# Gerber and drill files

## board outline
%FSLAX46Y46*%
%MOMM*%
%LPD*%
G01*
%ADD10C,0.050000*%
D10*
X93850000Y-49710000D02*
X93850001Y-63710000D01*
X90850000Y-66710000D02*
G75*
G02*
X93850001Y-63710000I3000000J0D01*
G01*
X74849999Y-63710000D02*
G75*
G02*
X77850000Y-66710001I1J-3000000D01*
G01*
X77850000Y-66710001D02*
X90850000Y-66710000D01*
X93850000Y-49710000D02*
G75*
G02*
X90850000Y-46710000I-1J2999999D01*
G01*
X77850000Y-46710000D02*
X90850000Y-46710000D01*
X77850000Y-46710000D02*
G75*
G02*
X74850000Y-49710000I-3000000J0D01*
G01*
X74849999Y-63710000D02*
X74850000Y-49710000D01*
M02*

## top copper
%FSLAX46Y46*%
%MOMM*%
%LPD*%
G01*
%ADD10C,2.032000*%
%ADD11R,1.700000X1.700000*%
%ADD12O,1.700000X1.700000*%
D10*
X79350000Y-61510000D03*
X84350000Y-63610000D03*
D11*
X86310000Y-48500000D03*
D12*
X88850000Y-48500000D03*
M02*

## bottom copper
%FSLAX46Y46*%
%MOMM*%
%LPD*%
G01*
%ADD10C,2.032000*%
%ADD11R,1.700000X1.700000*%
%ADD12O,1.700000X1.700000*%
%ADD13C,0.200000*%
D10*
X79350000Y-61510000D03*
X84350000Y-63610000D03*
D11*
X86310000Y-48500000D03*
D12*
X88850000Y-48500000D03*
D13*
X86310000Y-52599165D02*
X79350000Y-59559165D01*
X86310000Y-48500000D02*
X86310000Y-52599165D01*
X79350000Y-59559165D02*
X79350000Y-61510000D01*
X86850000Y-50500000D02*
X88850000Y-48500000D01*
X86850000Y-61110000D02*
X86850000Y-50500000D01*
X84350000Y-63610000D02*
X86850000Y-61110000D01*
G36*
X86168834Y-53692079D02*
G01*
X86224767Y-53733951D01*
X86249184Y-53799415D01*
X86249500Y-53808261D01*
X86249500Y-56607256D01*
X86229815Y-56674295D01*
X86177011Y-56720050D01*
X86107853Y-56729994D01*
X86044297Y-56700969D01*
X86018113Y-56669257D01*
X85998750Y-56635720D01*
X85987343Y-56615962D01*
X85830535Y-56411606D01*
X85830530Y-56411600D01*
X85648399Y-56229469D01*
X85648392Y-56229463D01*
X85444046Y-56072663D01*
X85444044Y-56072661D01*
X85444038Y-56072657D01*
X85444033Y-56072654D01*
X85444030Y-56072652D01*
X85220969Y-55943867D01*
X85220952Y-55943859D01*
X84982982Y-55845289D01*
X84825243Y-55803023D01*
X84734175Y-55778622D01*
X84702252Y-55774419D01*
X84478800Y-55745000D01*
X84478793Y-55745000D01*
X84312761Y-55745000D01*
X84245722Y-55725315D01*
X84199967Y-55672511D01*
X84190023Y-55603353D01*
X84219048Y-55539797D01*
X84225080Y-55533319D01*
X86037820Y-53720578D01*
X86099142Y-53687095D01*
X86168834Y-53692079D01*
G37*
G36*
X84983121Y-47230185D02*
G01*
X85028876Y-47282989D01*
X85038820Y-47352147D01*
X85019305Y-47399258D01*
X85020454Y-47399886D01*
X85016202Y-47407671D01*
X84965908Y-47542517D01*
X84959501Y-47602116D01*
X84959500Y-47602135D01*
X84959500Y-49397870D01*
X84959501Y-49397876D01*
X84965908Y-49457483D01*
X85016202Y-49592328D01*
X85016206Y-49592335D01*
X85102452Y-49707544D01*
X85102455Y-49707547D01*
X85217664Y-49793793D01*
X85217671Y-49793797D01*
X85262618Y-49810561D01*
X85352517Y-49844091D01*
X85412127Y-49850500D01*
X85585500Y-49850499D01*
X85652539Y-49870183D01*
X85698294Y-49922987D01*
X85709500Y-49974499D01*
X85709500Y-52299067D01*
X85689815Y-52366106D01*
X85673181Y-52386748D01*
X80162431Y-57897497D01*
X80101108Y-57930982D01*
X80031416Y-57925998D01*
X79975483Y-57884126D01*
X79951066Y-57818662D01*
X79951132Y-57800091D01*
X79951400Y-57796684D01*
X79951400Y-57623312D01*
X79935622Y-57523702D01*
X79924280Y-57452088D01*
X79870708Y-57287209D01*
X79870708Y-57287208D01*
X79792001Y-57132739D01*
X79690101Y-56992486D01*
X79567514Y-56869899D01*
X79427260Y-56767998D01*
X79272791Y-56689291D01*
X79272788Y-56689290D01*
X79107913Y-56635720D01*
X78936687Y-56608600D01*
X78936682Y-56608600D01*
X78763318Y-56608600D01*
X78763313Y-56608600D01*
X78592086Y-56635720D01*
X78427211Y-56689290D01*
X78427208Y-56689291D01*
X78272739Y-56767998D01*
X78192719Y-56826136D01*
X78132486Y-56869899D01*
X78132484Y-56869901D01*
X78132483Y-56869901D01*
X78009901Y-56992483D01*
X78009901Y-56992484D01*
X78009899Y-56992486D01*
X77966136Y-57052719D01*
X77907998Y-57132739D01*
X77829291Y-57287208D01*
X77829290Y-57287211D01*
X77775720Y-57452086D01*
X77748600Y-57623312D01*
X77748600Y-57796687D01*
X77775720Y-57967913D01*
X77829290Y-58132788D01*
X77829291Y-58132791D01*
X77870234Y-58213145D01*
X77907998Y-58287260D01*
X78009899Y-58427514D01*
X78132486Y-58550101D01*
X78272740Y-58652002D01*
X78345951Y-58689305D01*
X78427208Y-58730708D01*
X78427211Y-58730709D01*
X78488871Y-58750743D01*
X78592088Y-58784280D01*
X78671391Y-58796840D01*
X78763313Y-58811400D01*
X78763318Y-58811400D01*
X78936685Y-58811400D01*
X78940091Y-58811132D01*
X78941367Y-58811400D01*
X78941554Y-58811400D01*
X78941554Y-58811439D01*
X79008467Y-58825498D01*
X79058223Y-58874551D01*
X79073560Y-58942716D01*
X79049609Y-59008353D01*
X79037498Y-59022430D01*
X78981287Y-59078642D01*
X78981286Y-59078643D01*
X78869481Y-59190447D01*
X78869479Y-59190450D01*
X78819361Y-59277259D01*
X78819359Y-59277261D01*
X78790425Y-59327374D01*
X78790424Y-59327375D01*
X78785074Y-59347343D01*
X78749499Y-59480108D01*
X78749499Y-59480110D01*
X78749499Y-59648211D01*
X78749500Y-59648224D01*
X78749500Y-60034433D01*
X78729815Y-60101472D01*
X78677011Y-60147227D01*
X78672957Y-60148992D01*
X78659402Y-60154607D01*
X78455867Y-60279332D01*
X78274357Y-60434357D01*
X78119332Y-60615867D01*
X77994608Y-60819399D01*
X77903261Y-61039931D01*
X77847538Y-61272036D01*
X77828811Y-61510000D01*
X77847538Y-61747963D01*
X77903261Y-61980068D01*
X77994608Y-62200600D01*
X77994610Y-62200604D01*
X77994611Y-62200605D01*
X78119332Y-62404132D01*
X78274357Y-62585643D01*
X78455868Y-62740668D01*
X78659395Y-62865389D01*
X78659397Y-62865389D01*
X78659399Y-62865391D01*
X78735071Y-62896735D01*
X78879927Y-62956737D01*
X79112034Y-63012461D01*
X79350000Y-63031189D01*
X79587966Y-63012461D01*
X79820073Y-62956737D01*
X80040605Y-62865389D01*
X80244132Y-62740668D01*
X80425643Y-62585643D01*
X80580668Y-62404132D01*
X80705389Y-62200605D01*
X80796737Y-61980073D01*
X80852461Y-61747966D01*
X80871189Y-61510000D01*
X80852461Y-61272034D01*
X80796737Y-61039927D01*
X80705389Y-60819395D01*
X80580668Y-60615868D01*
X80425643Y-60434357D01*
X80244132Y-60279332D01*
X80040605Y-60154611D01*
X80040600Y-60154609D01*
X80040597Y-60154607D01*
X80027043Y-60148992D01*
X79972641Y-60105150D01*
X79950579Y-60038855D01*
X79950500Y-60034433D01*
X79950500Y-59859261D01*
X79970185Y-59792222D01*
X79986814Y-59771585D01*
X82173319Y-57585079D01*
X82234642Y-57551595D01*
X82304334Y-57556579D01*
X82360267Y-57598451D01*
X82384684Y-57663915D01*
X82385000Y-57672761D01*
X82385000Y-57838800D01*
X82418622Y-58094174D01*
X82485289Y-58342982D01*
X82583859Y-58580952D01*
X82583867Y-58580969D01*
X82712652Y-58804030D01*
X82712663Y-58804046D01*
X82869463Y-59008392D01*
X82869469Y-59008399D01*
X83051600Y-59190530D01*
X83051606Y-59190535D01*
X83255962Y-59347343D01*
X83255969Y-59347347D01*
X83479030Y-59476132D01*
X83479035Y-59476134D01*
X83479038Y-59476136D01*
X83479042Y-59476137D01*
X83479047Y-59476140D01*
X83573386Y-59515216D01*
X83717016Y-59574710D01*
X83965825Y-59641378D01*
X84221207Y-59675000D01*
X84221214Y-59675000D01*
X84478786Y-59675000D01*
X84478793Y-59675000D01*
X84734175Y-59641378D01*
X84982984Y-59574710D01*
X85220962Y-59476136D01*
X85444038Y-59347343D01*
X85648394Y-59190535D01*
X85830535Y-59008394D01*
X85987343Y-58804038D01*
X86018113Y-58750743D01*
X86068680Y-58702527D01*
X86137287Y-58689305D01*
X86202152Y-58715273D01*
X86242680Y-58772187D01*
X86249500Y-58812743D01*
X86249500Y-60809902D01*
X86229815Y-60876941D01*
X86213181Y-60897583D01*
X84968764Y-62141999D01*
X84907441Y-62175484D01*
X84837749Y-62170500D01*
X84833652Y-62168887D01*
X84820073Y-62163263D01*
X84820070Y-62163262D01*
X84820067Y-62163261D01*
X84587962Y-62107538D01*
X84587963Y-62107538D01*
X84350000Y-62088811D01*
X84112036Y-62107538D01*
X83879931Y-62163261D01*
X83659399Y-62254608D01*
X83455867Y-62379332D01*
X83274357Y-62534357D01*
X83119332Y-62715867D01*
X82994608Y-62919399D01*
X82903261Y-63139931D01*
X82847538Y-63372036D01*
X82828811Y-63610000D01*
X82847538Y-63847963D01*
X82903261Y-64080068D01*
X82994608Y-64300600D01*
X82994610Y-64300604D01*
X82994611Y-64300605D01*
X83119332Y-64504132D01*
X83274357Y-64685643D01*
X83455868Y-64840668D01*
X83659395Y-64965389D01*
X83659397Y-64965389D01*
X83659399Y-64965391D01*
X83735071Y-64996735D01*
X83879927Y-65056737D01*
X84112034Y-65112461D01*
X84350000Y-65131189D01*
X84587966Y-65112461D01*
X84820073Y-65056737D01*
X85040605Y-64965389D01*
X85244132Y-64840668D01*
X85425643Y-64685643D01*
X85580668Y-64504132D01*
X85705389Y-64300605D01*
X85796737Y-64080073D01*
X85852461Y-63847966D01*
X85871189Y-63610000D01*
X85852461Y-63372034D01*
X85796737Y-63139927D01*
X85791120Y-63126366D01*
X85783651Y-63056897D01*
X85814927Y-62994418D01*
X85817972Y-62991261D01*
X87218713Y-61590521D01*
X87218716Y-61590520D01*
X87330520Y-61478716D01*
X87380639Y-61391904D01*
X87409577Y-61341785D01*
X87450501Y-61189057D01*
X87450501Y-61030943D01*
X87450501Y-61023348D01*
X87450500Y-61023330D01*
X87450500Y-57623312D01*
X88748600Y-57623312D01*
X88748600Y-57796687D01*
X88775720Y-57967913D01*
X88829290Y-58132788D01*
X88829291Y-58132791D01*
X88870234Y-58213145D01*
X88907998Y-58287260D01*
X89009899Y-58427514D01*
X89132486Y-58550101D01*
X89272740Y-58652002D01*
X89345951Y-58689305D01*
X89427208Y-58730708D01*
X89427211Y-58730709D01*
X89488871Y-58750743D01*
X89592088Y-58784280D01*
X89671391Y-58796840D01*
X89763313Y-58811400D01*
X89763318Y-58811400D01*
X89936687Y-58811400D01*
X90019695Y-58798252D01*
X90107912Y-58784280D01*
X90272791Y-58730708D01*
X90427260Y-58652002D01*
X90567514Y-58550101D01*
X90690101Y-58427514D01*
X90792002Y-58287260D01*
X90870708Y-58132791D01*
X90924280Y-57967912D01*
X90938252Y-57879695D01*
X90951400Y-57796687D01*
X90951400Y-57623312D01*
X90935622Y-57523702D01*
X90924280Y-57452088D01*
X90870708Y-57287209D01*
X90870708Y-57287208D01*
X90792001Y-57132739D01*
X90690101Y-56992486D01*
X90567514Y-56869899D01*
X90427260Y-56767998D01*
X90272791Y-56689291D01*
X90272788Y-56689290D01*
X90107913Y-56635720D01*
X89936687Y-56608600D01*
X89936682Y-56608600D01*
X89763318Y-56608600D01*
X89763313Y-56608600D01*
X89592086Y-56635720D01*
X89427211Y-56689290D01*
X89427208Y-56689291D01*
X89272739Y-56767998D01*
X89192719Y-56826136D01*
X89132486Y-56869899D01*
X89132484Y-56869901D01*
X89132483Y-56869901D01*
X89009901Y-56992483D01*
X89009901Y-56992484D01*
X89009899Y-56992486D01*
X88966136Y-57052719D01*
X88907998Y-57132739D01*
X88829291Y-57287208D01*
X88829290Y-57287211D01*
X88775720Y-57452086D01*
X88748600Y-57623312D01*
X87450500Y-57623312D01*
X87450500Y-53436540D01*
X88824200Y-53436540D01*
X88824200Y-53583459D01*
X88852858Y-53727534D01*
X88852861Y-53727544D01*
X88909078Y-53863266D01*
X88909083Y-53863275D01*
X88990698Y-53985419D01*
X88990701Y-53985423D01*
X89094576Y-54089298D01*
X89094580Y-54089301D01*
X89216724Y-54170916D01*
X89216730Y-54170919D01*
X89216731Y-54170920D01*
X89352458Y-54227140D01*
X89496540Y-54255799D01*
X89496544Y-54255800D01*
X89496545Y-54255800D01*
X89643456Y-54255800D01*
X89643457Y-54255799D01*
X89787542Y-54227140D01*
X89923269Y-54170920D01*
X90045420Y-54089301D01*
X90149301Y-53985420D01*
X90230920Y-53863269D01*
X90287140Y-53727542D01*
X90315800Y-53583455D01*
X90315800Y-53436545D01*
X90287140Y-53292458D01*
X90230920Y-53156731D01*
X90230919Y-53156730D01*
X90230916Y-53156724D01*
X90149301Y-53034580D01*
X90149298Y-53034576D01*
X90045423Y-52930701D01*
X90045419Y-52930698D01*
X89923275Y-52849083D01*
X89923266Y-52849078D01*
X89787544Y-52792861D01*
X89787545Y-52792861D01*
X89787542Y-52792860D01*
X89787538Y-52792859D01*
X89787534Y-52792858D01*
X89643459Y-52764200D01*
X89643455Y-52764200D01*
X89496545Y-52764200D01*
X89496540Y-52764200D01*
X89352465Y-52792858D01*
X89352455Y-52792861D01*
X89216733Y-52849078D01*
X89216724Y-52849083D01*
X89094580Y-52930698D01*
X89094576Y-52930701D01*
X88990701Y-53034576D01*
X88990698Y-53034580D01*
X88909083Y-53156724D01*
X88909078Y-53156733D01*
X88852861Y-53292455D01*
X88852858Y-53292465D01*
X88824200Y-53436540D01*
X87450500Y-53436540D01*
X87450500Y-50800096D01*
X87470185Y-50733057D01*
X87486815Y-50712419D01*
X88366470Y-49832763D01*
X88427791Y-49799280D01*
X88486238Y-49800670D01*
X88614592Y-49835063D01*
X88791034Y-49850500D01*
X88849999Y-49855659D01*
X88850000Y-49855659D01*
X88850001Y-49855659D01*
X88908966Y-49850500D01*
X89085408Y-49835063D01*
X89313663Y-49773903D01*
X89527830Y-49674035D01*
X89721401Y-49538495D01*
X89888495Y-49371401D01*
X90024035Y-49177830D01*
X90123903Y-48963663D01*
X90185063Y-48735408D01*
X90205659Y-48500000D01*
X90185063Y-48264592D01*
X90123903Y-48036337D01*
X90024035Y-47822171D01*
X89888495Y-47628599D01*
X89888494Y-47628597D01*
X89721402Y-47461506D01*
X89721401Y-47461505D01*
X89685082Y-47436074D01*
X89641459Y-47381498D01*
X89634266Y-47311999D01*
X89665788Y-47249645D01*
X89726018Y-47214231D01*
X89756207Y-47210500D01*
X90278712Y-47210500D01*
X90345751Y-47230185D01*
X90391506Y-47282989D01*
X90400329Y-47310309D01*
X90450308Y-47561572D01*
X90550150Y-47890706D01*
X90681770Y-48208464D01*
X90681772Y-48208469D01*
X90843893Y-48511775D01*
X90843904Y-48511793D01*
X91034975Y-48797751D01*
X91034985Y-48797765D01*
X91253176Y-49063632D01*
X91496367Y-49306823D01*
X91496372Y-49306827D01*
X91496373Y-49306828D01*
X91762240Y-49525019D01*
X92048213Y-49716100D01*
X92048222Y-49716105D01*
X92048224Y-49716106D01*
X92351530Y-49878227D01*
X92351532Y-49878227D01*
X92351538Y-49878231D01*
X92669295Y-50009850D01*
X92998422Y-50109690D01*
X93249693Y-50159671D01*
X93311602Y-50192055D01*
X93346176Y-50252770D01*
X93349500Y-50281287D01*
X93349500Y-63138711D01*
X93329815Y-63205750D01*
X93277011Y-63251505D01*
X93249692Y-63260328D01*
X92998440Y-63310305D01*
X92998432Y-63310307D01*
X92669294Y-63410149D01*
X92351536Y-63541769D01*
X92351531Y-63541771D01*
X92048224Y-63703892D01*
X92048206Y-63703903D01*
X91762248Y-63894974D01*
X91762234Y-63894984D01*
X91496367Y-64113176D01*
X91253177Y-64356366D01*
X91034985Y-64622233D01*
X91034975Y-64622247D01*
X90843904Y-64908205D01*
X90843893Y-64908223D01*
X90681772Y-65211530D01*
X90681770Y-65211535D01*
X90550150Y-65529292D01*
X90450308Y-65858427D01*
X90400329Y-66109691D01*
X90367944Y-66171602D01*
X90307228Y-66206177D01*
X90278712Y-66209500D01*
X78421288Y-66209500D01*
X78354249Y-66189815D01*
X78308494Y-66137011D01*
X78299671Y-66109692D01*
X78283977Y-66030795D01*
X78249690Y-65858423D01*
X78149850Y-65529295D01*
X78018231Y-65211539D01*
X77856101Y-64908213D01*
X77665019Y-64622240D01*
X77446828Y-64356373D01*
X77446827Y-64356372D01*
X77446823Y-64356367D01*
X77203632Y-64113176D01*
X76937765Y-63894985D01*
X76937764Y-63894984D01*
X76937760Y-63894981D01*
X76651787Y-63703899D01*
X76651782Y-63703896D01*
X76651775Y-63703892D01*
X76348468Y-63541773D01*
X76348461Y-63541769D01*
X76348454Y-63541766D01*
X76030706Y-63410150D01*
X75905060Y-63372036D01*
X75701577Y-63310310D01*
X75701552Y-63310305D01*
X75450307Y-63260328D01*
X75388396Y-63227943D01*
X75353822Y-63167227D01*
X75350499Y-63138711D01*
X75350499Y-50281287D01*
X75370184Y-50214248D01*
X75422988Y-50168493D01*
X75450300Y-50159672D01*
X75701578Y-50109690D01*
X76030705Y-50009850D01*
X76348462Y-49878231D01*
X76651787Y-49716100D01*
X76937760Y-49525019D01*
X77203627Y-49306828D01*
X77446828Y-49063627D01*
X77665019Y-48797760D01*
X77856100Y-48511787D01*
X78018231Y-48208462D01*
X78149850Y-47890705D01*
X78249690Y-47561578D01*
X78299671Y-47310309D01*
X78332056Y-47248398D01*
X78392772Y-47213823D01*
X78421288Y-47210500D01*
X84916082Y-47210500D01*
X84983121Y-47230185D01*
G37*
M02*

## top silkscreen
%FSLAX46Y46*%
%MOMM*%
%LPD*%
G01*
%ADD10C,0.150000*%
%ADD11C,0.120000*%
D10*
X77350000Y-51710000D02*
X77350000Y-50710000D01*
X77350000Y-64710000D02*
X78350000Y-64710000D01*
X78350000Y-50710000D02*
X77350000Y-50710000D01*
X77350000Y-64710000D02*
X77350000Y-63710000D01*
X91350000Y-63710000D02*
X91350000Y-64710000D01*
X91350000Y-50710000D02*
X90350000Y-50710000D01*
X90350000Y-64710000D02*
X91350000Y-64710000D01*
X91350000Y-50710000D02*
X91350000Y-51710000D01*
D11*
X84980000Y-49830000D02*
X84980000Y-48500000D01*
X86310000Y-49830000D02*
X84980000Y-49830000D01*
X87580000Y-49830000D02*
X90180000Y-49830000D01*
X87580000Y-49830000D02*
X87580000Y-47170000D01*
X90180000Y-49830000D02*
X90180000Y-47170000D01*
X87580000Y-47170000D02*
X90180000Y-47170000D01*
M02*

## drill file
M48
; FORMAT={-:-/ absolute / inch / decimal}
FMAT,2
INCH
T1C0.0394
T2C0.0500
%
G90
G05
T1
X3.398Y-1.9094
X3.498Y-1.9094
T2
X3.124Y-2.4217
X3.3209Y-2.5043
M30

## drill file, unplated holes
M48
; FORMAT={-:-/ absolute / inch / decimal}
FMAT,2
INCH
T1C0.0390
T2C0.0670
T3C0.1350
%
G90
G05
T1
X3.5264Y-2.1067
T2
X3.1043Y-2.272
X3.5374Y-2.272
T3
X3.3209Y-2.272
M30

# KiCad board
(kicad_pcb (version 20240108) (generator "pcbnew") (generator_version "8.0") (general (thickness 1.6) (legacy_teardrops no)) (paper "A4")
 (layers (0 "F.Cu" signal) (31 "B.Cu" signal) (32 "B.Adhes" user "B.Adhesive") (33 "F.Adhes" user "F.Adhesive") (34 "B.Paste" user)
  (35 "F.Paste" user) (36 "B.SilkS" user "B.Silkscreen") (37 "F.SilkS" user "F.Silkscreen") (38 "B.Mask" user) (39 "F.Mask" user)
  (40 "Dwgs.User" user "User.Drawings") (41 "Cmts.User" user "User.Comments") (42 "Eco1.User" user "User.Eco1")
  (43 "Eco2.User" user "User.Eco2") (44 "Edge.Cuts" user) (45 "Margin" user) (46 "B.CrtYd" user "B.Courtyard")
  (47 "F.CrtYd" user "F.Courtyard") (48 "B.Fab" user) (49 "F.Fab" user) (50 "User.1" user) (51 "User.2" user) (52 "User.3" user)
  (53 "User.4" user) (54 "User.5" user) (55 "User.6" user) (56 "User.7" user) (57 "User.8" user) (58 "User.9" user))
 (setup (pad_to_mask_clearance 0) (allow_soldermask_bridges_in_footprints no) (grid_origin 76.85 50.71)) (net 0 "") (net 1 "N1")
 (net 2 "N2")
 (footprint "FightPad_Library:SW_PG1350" (layer "F.Cu") (at 84.35 57.71)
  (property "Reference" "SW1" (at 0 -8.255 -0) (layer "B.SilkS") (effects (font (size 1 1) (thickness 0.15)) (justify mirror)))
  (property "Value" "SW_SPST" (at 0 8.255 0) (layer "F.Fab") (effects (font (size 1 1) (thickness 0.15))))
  (fp_line (start -7 -6) (end -7 -7) (stroke (width 0.15) (type solid)) (layer "F.SilkS"))
  (fp_line (start -7 7) (end -7 6) (stroke (width 0.15) (type solid)) (layer "F.SilkS"))
  (fp_line (start -7 7) (end -6 7) (stroke (width 0.15) (type solid)) (layer "F.SilkS"))
  (fp_line (start -6 -7) (end -7 -7) (stroke (width 0.15) (type solid)) (layer "F.SilkS"))
  (fp_line (start 6 7) (end 7 7) (stroke (width 0.15) (type solid)) (layer "F.SilkS"))
  (fp_line (start 7 -7) (end 6 -7) (stroke (width 0.15) (type solid)) (layer "F.SilkS"))
  (fp_line (start 7 -7) (end 7 -6) (stroke (width 0.15) (type solid)) (layer "F.SilkS"))
  (fp_line (start 7 6) (end 7 7) (stroke (width 0.15) (type solid)) (layer "F.SilkS"))
  (pad "" np_thru_hole circle (at -5.5 0) (size 1.7018 1.7018) (drill 1.7018) (layers "*.Cu" "*.Mask"))
  (pad "" np_thru_hole circle (at 0 0) (size 3.429 3.429) (drill 3.429) (layers "*.Cu" "*.Mask"))
  (pad "" np_thru_hole circle (at 5.22 -4.2) (size 0.9906 0.9906) (drill 0.9906) (layers "*.Cu" "*.Mask"))
  (pad "" np_thru_hole circle (at 5.5 0) (size 1.7018 1.7018) (drill 1.7018) (layers "*.Cu" "*.Mask"))
  (pad "1" thru_hole circle (at 0 5.9) (size 2.032 2.032) (drill 1.27) (layers "*.Cu" "*.Mask") (remove_unused_layers no) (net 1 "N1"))
  (pad "2" thru_hole circle (at -5 3.8) (size 2.032 2.032) (drill 1.27) (layers "*.Cu" "*.Mask") (remove_unused_layers no) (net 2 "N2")))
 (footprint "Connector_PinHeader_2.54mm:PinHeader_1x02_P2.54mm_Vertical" (layer "F.Cu") (at 86.31 48.5 90)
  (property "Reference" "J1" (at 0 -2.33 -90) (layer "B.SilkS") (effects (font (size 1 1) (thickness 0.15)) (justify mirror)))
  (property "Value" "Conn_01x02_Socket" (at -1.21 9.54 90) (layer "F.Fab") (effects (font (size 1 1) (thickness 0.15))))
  (fp_line (start -1.33 -1.33) (end 0 -1.33) (stroke (width 0.12) (type solid)) (layer "F.SilkS"))
  (fp_line (start -1.33 0) (end -1.33 -1.33) (stroke (width 0.12) (type solid)) (layer "F.SilkS"))
  (fp_line (start 1.33 1.27) (end 1.33 3.87) (stroke (width 0.12) (type solid)) (layer "F.SilkS"))
  (fp_line (start -1.33 1.27) (end 1.33 1.27) (stroke (width 0.12) (type solid)) (layer "F.SilkS"))
  (fp_line (start -1.33 1.27) (end -1.33 3.87) (stroke (width 0.12) (type solid)) (layer "F.SilkS"))
  (fp_line (start -1.33 3.87) (end 1.33 3.87) (stroke (width 0.12) (type solid)) (layer "F.SilkS"))
  (pad "1" thru_hole rect (at 0 0 90) (size 1.7 1.7) (drill 1) (layers "*.Cu" "*.Mask") (remove_unused_layers no) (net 2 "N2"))
  (pad "2" thru_hole oval (at 0 2.54 90) (size 1.7 1.7) (drill 1) (layers "*.Cu" "*.Mask") (remove_unused_layers no) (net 1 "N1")))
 (gr_line (start 74.849999 63.71) (end 74.85 49.71) (stroke (width 0.05) (type default)) (layer "Edge.Cuts"))
 (gr_line (start 77.85 46.71) (end 90.85 46.71) (stroke (width 0.05) (type default)) (layer "Edge.Cuts"))
 (gr_arc (start 74.849999 63.71) (mid 76.97132 64.58868) (end 77.85 66.710001) (stroke (width 0.05) (type default)) (layer "Edge.Cuts"))
 (gr_line (start 77.85 66.710001) (end 90.85 66.71) (stroke (width 0.05) (type default)) (layer "Edge.Cuts"))
 (gr_arc (start 93.85 49.71) (mid 91.728679 48.831321) (end 90.85 46.71) (stroke (width 0.05) (type default)) (layer "Edge.Cuts"))
 (gr_arc (start 90.85 66.71) (mid 91.72868 64.588679) (end 93.850001 63.71) (stroke (width 0.05) (type default)) (layer "Edge.Cuts"))
 (gr_line (start 93.85 49.71) (end 93.850001 63.71) (stroke (width 0.05) (type default)) (layer "Edge.Cuts"))
 (gr_arc (start 77.85 46.71) (mid 76.97132 48.83132) (end 74.85 49.71) (stroke (width 0.05) (type default)) (layer "Edge.Cuts"))
 (segment (start 84.35 63.61) (end 86.85 61.11) (width 0.2) (layer "B.Cu") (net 1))
 (segment (start 86.85 61.11) (end 86.85 50.5) (width 0.2) (layer "B.Cu") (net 1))
 (segment (start 86.85 50.5) (end 88.85 48.5) (width 0.2) (layer "B.Cu") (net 1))
 (segment (start 79.35 59.559165) (end 79.35 61.51) (width 0.2) (layer "B.Cu") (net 2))
 (segment (start 86.31 52.599165) (end 79.35 59.559165) (width 0.2) (layer "B.Cu") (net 2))
 (segment (start 86.31 48.5) (end 86.31 52.599165) (width 0.2) (layer "B.Cu") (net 2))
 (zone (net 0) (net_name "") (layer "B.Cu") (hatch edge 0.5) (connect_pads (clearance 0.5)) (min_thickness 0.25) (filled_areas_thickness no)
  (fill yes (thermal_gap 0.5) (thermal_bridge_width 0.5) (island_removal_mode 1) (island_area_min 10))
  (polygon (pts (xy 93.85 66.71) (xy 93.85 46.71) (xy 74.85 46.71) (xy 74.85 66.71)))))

